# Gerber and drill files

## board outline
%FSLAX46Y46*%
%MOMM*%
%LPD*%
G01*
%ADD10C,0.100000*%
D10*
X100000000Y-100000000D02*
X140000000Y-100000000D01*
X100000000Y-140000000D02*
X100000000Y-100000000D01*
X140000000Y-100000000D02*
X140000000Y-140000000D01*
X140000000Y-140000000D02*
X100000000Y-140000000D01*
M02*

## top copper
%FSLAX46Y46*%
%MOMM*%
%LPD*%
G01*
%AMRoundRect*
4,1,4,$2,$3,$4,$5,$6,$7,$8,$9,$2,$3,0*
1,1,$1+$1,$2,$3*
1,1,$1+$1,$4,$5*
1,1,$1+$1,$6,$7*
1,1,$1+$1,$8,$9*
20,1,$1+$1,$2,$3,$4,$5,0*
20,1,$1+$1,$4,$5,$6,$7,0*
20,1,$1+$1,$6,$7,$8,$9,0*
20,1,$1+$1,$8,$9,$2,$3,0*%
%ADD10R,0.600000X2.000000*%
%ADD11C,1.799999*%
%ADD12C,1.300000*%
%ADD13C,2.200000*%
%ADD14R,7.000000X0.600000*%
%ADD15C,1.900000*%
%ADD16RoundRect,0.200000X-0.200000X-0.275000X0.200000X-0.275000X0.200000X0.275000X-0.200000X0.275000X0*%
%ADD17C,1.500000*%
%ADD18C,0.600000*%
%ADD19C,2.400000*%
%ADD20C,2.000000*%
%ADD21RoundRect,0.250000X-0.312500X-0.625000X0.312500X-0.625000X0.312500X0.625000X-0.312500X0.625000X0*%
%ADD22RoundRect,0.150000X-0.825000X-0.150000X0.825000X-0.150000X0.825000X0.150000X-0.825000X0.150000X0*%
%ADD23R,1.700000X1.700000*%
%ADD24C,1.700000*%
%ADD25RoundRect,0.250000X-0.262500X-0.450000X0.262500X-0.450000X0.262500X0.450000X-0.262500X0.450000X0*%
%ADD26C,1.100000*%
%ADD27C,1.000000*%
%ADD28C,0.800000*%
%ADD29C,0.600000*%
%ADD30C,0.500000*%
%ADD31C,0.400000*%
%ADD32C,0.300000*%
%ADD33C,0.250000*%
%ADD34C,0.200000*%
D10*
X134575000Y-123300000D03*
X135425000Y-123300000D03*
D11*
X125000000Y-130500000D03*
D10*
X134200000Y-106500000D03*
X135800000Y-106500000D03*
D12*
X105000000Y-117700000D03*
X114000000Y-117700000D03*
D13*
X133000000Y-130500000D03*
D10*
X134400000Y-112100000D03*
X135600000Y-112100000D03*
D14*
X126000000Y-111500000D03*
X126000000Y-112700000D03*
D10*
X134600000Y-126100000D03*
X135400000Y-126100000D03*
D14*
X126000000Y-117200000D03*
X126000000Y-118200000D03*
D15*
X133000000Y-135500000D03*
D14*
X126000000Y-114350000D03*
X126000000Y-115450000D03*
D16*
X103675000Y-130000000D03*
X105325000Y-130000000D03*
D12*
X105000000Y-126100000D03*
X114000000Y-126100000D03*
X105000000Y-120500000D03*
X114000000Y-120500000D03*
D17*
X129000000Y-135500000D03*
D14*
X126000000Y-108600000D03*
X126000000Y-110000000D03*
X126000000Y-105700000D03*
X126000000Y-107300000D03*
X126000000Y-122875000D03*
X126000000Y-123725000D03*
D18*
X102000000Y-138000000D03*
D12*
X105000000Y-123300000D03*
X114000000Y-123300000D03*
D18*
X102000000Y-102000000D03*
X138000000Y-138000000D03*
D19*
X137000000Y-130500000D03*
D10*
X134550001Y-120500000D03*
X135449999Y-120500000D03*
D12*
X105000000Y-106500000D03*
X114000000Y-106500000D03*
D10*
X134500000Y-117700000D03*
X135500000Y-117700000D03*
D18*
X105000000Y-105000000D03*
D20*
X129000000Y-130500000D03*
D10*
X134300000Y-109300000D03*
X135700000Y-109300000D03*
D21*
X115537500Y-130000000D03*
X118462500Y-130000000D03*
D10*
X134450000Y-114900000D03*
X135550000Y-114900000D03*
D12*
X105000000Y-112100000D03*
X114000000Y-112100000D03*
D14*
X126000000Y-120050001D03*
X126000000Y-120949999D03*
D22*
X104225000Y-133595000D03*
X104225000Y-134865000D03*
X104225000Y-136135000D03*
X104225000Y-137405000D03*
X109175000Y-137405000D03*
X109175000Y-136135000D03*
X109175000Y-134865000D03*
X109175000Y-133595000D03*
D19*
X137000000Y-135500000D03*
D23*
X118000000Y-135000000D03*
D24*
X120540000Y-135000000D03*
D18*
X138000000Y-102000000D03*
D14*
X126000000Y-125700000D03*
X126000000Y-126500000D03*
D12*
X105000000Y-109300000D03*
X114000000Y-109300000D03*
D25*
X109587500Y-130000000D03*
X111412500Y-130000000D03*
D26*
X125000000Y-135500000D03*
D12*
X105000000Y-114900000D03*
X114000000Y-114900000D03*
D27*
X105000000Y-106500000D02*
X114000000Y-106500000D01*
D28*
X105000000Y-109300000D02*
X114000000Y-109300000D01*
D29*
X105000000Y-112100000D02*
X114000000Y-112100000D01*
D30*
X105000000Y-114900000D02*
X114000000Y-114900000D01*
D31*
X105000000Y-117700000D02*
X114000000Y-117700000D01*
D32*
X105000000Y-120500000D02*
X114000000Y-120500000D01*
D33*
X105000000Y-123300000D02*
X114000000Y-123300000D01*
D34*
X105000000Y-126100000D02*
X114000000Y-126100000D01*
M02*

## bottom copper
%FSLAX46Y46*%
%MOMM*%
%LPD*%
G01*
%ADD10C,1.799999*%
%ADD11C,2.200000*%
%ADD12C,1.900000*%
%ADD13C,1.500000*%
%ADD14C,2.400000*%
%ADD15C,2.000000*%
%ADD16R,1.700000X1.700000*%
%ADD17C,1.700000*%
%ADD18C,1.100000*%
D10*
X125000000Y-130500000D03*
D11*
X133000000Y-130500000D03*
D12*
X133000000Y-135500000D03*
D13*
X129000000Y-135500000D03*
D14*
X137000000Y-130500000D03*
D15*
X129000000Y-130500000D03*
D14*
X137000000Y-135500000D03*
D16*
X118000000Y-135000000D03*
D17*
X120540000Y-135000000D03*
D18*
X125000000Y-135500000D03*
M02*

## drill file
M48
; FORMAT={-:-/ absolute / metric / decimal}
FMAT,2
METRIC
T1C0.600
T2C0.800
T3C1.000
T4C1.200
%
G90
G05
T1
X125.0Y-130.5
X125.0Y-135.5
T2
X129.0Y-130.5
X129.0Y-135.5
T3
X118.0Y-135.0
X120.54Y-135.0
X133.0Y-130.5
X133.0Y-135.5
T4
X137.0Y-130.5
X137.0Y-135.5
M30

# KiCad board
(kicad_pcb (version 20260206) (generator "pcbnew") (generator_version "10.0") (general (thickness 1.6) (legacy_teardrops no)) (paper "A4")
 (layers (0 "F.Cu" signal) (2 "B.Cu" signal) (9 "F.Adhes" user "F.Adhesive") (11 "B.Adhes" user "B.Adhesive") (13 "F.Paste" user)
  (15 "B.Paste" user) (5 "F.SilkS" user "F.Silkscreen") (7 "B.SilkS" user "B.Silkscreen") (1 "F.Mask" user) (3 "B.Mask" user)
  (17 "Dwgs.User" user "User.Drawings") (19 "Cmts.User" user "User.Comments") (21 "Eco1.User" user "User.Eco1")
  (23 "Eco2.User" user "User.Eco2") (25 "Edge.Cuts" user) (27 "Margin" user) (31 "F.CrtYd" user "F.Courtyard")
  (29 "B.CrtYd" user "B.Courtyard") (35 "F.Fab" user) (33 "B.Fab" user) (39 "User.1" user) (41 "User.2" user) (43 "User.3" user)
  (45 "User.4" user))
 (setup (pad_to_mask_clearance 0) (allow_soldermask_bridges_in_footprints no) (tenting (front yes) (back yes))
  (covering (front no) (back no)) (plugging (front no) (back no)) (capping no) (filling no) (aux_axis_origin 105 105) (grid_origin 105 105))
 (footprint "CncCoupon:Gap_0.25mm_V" (layer "F.Cu") (at 135 123.3)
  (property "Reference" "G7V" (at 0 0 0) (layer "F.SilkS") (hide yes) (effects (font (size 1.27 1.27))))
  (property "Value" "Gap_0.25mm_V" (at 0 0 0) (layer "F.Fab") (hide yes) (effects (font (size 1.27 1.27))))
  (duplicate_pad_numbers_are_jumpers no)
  (pad "1" smd rect (at -0.425 0) (size 0.6 2) (layers "F.Cu" "F.Mask") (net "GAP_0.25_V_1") (thermal_bridge_angle 45))
  (pad "2" smd rect (at 0.425 0) (size 0.6 2) (layers "F.Cu" "F.Mask") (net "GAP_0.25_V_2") (thermal_bridge_angle 45)))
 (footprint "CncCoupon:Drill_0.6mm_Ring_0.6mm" (layer "F.Cu") (at 125 130.5)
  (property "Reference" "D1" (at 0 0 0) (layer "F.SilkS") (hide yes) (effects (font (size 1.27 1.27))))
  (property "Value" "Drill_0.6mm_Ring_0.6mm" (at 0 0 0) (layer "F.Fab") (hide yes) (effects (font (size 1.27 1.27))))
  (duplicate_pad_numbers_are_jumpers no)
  (pad "1" thru_hole circle (at 0 0) (size 1.799999 1.799999) (drill 0.6) (layers "*.Cu" "*.Mask") (remove_unused_layers no)
   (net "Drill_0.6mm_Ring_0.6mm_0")))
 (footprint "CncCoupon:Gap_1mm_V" (layer "F.Cu") (at 135 106.5)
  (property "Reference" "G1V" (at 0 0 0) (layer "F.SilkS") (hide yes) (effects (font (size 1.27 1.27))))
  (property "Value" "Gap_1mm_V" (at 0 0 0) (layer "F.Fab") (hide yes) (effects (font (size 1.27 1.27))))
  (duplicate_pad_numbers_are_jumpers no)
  (pad "1" smd rect (at -0.8 0) (size 0.6 2) (layers "F.Cu" "F.Mask") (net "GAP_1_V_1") (thermal_bridge_angle 45))
  (pad "2" smd rect (at 0.8 0) (size 0.6 2) (layers "F.Cu" "F.Mask") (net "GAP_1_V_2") (thermal_bridge_angle 45)))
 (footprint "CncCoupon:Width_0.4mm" (layer "F.Cu") (at 109.5 117.7)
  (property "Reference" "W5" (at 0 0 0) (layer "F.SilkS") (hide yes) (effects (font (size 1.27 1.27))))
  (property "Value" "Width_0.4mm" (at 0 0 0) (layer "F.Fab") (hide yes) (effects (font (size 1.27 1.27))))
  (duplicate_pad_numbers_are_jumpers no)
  (pad "1" smd circle (at -4.5 0) (size 1.3 1.3) (layers "F.Cu" "F.Mask") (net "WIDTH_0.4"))
  (pad "2" smd circle (at 4.5 0) (size 1.3 1.3) (layers "F.Cu" "F.Mask") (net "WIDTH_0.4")))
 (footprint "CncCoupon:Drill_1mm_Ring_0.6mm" (layer "F.Cu") (at 133 130.5)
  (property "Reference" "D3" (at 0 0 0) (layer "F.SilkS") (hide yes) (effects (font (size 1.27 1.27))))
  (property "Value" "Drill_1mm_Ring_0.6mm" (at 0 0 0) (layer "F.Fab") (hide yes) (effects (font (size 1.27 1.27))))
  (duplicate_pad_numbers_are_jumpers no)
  (pad "1" thru_hole circle (at 0 0) (size 2.2 2.2) (drill 1) (layers "*.Cu" "*.Mask") (remove_unused_layers no)
   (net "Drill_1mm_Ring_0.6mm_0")))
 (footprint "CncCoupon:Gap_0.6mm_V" (layer "F.Cu") (at 135 112.1)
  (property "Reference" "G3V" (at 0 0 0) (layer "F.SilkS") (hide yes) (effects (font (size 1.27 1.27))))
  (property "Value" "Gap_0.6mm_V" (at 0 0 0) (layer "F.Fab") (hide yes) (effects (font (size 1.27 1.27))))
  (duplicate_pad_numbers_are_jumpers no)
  (pad "1" smd rect (at -0.6 0) (size 0.6 2) (layers "F.Cu" "F.Mask") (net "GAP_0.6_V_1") (thermal_bridge_angle 45))
  (pad "2" smd rect (at 0.6 0) (size 0.6 2) (layers "F.Cu" "F.Mask") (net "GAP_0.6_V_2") (thermal_bridge_angle 45)))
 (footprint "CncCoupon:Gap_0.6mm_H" (layer "F.Cu") (at 126 112.1)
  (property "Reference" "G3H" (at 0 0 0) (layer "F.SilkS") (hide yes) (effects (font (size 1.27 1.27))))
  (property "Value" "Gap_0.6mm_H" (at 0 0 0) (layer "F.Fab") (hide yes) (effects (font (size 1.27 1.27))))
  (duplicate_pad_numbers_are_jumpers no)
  (pad "1" smd rect (at 0 -0.6) (size 7 0.6) (layers "F.Cu" "F.Mask") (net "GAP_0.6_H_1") (thermal_bridge_angle 45))
  (pad "2" smd rect (at 0 0.6) (size 7 0.6) (layers "F.Cu" "F.Mask") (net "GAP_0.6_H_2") (thermal_bridge_angle 45)))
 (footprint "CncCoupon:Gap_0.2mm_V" (layer "F.Cu") (at 135 126.1)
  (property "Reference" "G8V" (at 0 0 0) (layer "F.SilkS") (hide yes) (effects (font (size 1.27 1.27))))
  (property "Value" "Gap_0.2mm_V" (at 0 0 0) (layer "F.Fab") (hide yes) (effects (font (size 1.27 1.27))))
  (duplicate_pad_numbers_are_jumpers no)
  (pad "1" smd rect (at -0.4 0) (size 0.6 2) (layers "F.Cu" "F.Mask") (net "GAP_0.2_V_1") (thermal_bridge_angle 45))
  (pad "2" smd rect (at 0.4 0) (size 0.6 2) (layers "F.Cu" "F.Mask") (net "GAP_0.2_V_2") (thermal_bridge_angle 45)))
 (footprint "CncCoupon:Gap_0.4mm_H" (layer "F.Cu") (at 126 117.7)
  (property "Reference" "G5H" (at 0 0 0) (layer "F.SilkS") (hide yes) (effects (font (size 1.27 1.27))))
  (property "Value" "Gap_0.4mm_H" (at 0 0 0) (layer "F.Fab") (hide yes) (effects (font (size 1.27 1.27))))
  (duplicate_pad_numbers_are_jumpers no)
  (pad "1" smd rect (at 0 -0.5) (size 7 0.6) (layers "F.Cu" "F.Mask") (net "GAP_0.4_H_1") (thermal_bridge_angle 45))
  (pad "2" smd rect (at 0 0.5) (size 7 0.6) (layers "F.Cu" "F.Mask") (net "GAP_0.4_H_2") (thermal_bridge_angle 45)))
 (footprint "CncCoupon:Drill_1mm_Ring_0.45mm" (layer "F.Cu") (at 133 135.5)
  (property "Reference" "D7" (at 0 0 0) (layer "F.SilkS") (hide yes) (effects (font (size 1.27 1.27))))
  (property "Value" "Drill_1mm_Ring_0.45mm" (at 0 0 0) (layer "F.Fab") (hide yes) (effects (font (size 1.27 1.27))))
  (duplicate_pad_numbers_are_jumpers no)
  (pad "1" thru_hole circle (at 0 0) (size 1.9 1.9) (drill 1) (layers "*.Cu" "*.Mask") (remove_unused_layers no)
   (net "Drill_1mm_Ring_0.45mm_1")))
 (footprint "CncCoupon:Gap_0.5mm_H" (layer "F.Cu") (at 126 114.9)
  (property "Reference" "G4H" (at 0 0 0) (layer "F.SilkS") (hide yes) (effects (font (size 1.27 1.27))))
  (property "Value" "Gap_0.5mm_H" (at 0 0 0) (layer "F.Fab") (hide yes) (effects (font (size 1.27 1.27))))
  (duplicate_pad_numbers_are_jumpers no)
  (pad "1" smd rect (at 0 -0.55) (size 7 0.6) (layers "F.Cu" "F.Mask") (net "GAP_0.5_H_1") (thermal_bridge_angle 45))
  (pad "2" smd rect (at 0 0.55) (size 7 0.6) (layers "F.Cu" "F.Mask") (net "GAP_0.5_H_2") (thermal_bridge_angle 45)))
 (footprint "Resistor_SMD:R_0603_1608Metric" (layer "F.Cu") (at 104.5 130)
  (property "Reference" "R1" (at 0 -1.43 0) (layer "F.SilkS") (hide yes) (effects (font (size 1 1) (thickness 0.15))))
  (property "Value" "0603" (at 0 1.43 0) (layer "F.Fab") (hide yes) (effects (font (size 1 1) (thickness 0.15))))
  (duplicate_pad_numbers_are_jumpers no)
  (pad "1" smd roundrect (at -0.825 0) (size 0.8 0.95) (layers "F.Cu" "F.Mask" "F.Paste") (roundrect_rratio 0.25) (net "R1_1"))
  (pad "2" smd roundrect (at 0.825 0) (size 0.8 0.95) (layers "F.Cu" "F.Mask" "F.Paste") (roundrect_rratio 0.25) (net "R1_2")))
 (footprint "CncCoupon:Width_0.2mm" (layer "F.Cu") (at 109.5 126.1)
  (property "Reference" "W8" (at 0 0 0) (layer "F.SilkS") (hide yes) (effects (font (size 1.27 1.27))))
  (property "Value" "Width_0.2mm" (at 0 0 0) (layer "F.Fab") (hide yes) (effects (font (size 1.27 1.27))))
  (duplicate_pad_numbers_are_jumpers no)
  (pad "1" smd circle (at -4.5 0) (size 1.3 1.3) (layers "F.Cu" "F.Mask") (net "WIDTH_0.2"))
  (pad "2" smd circle (at 4.5 0) (size 1.3 1.3) (layers "F.Cu" "F.Mask") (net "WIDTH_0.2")))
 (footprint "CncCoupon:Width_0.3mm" (layer "F.Cu") (at 109.5 120.5)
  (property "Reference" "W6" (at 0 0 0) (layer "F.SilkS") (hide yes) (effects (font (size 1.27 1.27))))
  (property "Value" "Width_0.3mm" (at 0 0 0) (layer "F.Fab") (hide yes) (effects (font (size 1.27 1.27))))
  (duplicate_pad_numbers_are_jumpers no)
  (pad "1" smd circle (at -4.5 0) (size 1.3 1.3) (layers "F.Cu" "F.Mask") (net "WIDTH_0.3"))
  (pad "2" smd circle (at 4.5 0) (size 1.3 1.3) (layers "F.Cu" "F.Mask") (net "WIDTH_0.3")))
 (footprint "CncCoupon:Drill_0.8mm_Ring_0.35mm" (layer "F.Cu") (at 129 135.5)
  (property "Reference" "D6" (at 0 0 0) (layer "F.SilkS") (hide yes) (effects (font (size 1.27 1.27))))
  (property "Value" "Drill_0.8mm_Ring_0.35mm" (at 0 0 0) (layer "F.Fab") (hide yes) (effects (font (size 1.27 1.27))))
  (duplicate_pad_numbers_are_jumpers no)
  (pad "1" thru_hole circle (at 0 0) (size 1.5 1.5) (drill 0.8) (layers "*.Cu" "*.Mask") (remove_unused_layers no)
   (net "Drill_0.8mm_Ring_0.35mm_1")))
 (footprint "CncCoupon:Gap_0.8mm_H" (layer "F.Cu") (at 126 109.3)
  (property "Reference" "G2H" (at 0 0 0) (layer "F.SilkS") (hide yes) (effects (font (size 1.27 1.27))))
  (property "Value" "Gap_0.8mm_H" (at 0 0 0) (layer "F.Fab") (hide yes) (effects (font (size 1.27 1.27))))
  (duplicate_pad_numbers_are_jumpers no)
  (pad "1" smd rect (at 0 -0.7) (size 7 0.6) (layers "F.Cu" "F.Mask") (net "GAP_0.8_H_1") (thermal_bridge_angle 45))
  (pad "2" smd rect (at 0 0.7) (size 7 0.6) (layers "F.Cu" "F.Mask") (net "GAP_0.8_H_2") (thermal_bridge_angle 45)))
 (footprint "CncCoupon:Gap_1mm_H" (layer "F.Cu") (at 126 106.5)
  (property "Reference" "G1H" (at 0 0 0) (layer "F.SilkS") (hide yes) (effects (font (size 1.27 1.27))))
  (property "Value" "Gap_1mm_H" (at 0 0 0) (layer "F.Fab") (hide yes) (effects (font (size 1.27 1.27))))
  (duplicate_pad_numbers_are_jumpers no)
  (pad "1" smd rect (at 0 -0.8) (size 7 0.6) (layers "F.Cu" "F.Mask") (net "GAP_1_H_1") (thermal_bridge_angle 45))
  (pad "2" smd rect (at 0 0.8) (size 7 0.6) (layers "F.Cu" "F.Mask") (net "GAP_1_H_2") (thermal_bridge_angle 45)))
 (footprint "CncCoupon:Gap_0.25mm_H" (layer "F.Cu") (at 126 123.3)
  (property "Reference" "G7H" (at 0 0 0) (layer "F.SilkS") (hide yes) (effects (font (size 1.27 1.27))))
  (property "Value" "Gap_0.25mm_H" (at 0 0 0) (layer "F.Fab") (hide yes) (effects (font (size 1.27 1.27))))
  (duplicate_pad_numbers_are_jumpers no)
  (pad "1" smd rect (at 0 -0.425) (size 7 0.6) (layers "F.Cu" "F.Mask") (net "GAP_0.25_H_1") (thermal_bridge_angle 45))
  (pad "2" smd rect (at 0 0.425) (size 7 0.6) (layers "F.Cu" "F.Mask") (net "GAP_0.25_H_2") (thermal_bridge_angle 45)))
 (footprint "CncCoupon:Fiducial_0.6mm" (layer "F.Cu") (at 102 138)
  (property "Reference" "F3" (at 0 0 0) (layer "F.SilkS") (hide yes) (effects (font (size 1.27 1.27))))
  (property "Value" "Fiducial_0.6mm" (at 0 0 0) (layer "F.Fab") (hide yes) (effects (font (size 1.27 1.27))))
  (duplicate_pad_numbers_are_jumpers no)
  (pad "1" smd circle (at 0 0) (size 0.6 0.6) (layers "F.Cu" "F.Mask") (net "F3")))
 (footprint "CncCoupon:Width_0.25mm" (layer "F.Cu") (at 109.5 123.3)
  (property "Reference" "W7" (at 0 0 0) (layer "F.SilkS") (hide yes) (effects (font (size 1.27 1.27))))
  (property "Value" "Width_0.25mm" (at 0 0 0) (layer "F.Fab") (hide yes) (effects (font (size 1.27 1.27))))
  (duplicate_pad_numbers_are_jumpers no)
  (pad "1" smd circle (at -4.5 0) (size 1.3 1.3) (layers "F.Cu" "F.Mask") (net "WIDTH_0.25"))
  (pad "2" smd circle (at 4.5 0) (size 1.3 1.3) (layers "F.Cu" "F.Mask") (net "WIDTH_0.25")))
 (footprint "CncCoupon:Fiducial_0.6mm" (layer "F.Cu") (at 102 102)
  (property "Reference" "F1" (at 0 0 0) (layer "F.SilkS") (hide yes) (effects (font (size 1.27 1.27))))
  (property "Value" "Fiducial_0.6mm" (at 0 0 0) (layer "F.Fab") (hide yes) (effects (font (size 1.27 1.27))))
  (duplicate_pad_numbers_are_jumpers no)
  (pad "1" smd circle (at 0 0) (size 0.6 0.6) (layers "F.Cu" "F.Mask") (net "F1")))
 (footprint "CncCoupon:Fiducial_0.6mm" (layer "F.Cu") (at 138 138)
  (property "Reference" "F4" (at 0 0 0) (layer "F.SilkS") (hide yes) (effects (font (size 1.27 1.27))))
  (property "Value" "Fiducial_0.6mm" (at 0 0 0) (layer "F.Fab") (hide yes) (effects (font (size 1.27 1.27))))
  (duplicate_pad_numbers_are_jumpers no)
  (pad "1" smd circle (at 0 0) (size 0.6 0.6) (layers "F.Cu" "F.Mask") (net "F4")))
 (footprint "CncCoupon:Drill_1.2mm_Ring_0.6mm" (layer "F.Cu") (at 137 130.5)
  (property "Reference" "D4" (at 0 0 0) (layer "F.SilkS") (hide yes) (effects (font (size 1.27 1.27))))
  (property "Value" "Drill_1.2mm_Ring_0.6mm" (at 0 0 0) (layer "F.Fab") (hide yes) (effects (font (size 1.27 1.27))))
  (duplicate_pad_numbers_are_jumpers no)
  (pad "1" thru_hole circle (at 0 0) (size 2.4 2.4) (drill 1.2) (layers "*.Cu" "*.Mask") (remove_unused_layers no)
   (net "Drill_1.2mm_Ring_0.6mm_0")))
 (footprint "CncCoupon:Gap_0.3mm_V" (layer "F.Cu") (at 135 120.5)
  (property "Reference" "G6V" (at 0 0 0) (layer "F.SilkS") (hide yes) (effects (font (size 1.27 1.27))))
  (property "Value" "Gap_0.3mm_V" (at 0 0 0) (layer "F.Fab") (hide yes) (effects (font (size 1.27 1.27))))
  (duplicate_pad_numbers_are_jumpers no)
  (pad "1" smd rect (at -0.449999 0) (size 0.6 2) (layers "F.Cu" "F.Mask") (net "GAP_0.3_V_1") (thermal_bridge_angle 45))
  (pad "2" smd rect (at 0.449999 0) (size 0.6 2) (layers "F.Cu" "F.Mask") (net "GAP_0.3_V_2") (thermal_bridge_angle 45)))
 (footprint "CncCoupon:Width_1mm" (layer "F.Cu") (at 109.5 106.5)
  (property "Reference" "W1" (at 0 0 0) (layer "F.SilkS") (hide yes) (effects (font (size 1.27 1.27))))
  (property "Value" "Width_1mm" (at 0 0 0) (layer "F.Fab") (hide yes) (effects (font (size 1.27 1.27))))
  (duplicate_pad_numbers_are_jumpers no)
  (pad "1" smd circle (at -4.5 0) (size 1.3 1.3) (layers "F.Cu" "F.Mask") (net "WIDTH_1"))
  (pad "2" smd circle (at 4.5 0) (size 1.3 1.3) (layers "F.Cu" "F.Mask") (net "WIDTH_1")))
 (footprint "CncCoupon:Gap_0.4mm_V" (layer "F.Cu") (at 135 117.7)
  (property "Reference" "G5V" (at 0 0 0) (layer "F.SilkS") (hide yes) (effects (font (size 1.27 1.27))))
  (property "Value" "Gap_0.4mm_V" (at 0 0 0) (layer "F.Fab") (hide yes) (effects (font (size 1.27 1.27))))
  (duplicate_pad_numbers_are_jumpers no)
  (pad "1" smd rect (at -0.5 0) (size 0.6 2) (layers "F.Cu" "F.Mask") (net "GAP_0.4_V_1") (thermal_bridge_angle 45))
  (pad "2" smd rect (at 0.5 0) (size 0.6 2) (layers "F.Cu" "F.Mask") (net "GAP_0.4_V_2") (thermal_bridge_angle 45)))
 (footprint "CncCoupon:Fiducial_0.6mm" (layer "F.Cu") (at 105 105)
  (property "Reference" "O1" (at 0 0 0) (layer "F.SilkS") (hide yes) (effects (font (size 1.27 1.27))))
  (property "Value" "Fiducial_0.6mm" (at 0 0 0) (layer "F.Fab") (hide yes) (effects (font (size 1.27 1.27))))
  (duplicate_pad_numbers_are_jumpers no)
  (pad "1" smd circle (at 0 0) (size 0.6 0.6) (layers "F.Cu" "F.Mask") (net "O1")))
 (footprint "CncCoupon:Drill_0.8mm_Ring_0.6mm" (layer "F.Cu") (at 129 130.5)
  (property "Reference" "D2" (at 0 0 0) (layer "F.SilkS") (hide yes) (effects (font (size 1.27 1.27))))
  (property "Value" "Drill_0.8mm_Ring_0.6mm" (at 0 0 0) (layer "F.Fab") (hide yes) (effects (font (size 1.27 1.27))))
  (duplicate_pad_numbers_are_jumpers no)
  (pad "1" thru_hole circle (at 0 0) (size 2 2) (drill 0.8) (layers "*.Cu" "*.Mask") (remove_unused_layers no)
   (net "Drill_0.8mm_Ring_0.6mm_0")))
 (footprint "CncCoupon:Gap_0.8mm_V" (layer "F.Cu") (at 135 109.3)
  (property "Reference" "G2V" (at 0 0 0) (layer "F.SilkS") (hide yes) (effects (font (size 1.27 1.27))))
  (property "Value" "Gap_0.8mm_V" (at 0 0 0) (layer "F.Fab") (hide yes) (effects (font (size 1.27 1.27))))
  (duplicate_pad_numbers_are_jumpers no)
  (pad "1" smd rect (at -0.7 0) (size 0.6 2) (layers "F.Cu" "F.Mask") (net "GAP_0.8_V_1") (thermal_bridge_angle 45))
  (pad "2" smd rect (at 0.7 0) (size 0.6 2) (layers "F.Cu" "F.Mask") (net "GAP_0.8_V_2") (thermal_bridge_angle 45)))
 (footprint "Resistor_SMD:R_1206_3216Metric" (layer "F.Cu") (at 117 130)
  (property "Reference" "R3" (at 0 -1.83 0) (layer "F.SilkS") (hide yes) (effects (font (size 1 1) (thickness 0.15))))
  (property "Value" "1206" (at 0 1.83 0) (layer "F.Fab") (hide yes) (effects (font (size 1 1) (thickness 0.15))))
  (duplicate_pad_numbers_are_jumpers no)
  (pad "1" smd roundrect (at -1.4625 0) (size 1.125 1.75) (layers "F.Cu" "F.Mask" "F.Paste") (roundrect_rratio 0.222222) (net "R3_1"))
  (pad "2" smd roundrect (at 1.4625 0) (size 1.125 1.75) (layers "F.Cu" "F.Mask" "F.Paste") (roundrect_rratio 0.222222) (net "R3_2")))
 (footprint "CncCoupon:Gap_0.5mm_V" (layer "F.Cu") (at 135 114.9)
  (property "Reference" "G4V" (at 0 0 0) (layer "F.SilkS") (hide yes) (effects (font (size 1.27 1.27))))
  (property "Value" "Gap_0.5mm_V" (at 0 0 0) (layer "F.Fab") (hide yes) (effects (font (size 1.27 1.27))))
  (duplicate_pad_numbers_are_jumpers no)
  (pad "1" smd rect (at -0.55 0) (size 0.6 2) (layers "F.Cu" "F.Mask") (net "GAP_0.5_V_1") (thermal_bridge_angle 45))
  (pad "2" smd rect (at 0.55 0) (size 0.6 2) (layers "F.Cu" "F.Mask") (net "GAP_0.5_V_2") (thermal_bridge_angle 45)))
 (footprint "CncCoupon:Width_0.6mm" (layer "F.Cu") (at 109.5 112.1)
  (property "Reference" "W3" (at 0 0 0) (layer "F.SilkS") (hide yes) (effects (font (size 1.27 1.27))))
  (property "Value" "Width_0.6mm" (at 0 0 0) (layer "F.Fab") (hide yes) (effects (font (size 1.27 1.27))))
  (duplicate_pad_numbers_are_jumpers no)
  (pad "1" smd circle (at -4.5 0) (size 1.3 1.3) (layers "F.Cu" "F.Mask") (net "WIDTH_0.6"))
  (pad "2" smd circle (at 4.5 0) (size 1.3 1.3) (layers "F.Cu" "F.Mask") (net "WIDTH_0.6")))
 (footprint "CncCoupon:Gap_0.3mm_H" (layer "F.Cu") (at 126 120.5)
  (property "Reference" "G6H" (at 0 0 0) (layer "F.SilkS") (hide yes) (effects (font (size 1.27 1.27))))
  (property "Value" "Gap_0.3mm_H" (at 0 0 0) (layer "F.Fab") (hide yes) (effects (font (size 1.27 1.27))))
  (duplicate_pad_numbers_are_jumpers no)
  (pad "1" smd rect (at 0 -0.449999) (size 7 0.6) (layers "F.Cu" "F.Mask") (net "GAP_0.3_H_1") (thermal_bridge_angle 45))
  (pad "2" smd rect (at 0 0.449999) (size 7 0.6) (layers "F.Cu" "F.Mask") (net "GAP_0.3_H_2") (thermal_bridge_angle 45)))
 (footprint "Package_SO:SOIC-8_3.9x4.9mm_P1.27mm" (layer "F.Cu") (at 106.7 135.5)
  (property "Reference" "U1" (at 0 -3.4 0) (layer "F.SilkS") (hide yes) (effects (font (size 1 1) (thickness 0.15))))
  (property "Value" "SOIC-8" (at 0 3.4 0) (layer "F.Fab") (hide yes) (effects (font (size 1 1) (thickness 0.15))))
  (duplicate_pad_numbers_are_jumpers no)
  (pad "1" smd roundrect (at -2.475 -1.905) (size 1.95 0.6) (layers "F.Cu" "F.Mask" "F.Paste") (roundrect_rratio 0.25) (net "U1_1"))
  (pad "2" smd roundrect (at -2.475 -0.635) (size 1.95 0.6) (layers "F.Cu" "F.Mask" "F.Paste") (roundrect_rratio 0.25) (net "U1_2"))
  (pad "3" smd roundrect (at -2.475 0.635) (size 1.95 0.6) (layers "F.Cu" "F.Mask" "F.Paste") (roundrect_rratio 0.25) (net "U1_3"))
  (pad "4" smd roundrect (at -2.475 1.905) (size 1.95 0.6) (layers "F.Cu" "F.Mask" "F.Paste") (roundrect_rratio 0.25) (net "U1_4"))
  (pad "5" smd roundrect (at 2.475 1.905) (size 1.95 0.6) (layers "F.Cu" "F.Mask" "F.Paste") (roundrect_rratio 0.25) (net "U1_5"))
  (pad "6" smd roundrect (at 2.475 0.635) (size 1.95 0.6) (layers "F.Cu" "F.Mask" "F.Paste") (roundrect_rratio 0.25) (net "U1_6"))
  (pad "7" smd roundrect (at 2.475 -0.635) (size 1.95 0.6) (layers "F.Cu" "F.Mask" "F.Paste") (roundrect_rratio 0.25) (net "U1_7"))
  (pad "8" smd roundrect (at 2.475 -1.905) (size 1.95 0.6) (layers "F.Cu" "F.Mask" "F.Paste") (roundrect_rratio 0.25) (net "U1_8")))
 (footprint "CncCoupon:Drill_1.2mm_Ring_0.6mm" (layer "F.Cu") (at 137 135.5)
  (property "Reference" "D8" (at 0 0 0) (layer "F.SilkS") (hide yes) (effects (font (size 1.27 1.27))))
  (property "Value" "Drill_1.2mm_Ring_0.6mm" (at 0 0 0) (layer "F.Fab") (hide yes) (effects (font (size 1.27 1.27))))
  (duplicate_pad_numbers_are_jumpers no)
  (pad "1" thru_hole circle (at 0 0) (size 2.4 2.4) (drill 1.2) (layers "*.Cu" "*.Mask") (remove_unused_layers no)
   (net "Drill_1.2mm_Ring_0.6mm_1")))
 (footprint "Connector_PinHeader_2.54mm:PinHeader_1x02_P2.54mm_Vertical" (layer "F.Cu") (at 118 135 90)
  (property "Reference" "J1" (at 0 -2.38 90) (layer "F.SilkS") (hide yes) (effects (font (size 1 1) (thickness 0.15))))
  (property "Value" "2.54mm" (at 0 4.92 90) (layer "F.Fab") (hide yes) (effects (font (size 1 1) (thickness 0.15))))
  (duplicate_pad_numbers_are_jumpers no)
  (pad "1" thru_hole rect (at 0 0 90) (size 1.7 1.7) (drill 1) (layers "*.Cu" "*.Mask") (remove_unused_layers no) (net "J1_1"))
  (pad "2" thru_hole circle (at 0 2.54 90) (size 1.7 1.7) (drill 1) (layers "*.Cu" "*.Mask") (remove_unused_layers no) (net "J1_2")))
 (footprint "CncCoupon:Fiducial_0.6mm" (layer "F.Cu") (at 138 102)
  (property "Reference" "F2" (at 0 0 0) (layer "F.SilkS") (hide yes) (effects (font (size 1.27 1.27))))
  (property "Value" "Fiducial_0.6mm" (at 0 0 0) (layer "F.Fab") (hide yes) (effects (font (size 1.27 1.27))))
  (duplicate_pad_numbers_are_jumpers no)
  (pad "1" smd circle (at 0 0) (size 0.6 0.6) (layers "F.Cu" "F.Mask") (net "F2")))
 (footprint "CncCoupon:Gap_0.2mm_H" (layer "F.Cu") (at 126 126.1)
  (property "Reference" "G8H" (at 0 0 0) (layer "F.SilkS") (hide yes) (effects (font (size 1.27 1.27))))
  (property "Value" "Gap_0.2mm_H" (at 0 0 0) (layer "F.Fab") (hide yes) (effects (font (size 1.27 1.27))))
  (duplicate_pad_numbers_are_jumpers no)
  (pad "1" smd rect (at 0 -0.4) (size 7 0.6) (layers "F.Cu" "F.Mask") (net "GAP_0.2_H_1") (thermal_bridge_angle 45))
  (pad "2" smd rect (at 0 0.4) (size 7 0.6) (layers "F.Cu" "F.Mask") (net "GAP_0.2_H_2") (thermal_bridge_angle 45)))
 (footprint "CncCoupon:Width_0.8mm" (layer "F.Cu") (at 109.5 109.3)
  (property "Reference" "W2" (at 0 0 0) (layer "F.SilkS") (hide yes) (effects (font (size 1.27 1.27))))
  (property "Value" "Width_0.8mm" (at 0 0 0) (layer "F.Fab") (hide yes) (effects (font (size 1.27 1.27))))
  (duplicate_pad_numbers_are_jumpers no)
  (pad "1" smd circle (at -4.5 0) (size 1.3 1.3) (layers "F.Cu" "F.Mask") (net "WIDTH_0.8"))
  (pad "2" smd circle (at 4.5 0) (size 1.3 1.3) (layers "F.Cu" "F.Mask") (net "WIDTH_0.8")))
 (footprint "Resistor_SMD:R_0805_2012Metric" (layer "F.Cu") (at 110.5 130)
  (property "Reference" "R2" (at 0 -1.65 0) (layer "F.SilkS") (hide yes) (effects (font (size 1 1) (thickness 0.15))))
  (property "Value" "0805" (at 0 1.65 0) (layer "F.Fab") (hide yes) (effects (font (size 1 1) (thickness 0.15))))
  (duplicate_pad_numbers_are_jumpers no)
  (pad "1" smd roundrect (at -0.9125 0) (size 1.025 1.4) (layers "F.Cu" "F.Mask" "F.Paste") (roundrect_rratio 0.243902) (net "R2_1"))
  (pad "2" smd roundrect (at 0.9125 0) (size 1.025 1.4) (layers "F.Cu" "F.Mask" "F.Paste") (roundrect_rratio 0.243902) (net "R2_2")))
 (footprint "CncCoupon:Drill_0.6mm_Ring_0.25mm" (layer "F.Cu") (at 125 135.5)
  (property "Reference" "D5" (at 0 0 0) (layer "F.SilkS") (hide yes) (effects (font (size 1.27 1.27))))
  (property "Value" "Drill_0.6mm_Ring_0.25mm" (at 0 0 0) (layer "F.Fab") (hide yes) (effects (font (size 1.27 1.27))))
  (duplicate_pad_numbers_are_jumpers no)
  (pad "1" thru_hole circle (at 0 0) (size 1.1 1.1) (drill 0.6) (layers "*.Cu" "*.Mask") (remove_unused_layers no)
   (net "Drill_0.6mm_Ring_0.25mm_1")))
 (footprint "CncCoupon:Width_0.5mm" (layer "F.Cu") (at 109.5 114.9)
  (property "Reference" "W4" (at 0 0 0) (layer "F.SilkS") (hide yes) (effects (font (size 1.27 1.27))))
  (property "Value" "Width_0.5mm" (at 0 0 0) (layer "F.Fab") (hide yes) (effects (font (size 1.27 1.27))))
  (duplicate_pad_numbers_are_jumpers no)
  (pad "1" smd circle (at -4.5 0) (size 1.3 1.3) (layers "F.Cu" "F.Mask") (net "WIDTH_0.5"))
  (pad "2" smd circle (at 4.5 0) (size 1.3 1.3) (layers "F.Cu" "F.Mask") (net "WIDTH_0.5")))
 (gr_line (start 100 100) (end 140 100) (stroke (width 0.1) (type default)) (layer "Edge.Cuts"))
 (gr_line (start 100 140) (end 100 100) (stroke (width 0.1) (type default)) (layer "Edge.Cuts"))
 (gr_line (start 140 100) (end 140 140) (stroke (width 0.1) (type default)) (layer "Edge.Cuts"))
 (gr_line (start 140 140) (end 100 140) (stroke (width 0.1) (type default)) (layer "Edge.Cuts"))
 (segment (start 105 106.5) (end 114 106.5) (width 1) (layer "F.Cu") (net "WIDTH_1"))
 (segment (start 105 109.3) (end 114 109.3) (width 0.8) (layer "F.Cu") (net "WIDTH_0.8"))
 (segment (start 105 112.1) (end 114 112.1) (width 0.6) (layer "F.Cu") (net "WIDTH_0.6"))
 (segment (start 105 114.9) (end 114 114.9) (width 0.5) (layer "F.Cu") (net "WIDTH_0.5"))
 (segment (start 105 117.7) (end 114 117.7) (width 0.4) (layer "F.Cu") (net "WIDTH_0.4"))
 (segment (start 105 120.5) (end 114 120.5) (width 0.3) (layer "F.Cu") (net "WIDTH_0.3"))
 (segment (start 105 123.3) (end 114 123.3) (width 0.25) (layer "F.Cu") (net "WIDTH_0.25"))
 (segment (start 105 126.1) (end 114 126.1) (width 0.2) (layer "F.Cu") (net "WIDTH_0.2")))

